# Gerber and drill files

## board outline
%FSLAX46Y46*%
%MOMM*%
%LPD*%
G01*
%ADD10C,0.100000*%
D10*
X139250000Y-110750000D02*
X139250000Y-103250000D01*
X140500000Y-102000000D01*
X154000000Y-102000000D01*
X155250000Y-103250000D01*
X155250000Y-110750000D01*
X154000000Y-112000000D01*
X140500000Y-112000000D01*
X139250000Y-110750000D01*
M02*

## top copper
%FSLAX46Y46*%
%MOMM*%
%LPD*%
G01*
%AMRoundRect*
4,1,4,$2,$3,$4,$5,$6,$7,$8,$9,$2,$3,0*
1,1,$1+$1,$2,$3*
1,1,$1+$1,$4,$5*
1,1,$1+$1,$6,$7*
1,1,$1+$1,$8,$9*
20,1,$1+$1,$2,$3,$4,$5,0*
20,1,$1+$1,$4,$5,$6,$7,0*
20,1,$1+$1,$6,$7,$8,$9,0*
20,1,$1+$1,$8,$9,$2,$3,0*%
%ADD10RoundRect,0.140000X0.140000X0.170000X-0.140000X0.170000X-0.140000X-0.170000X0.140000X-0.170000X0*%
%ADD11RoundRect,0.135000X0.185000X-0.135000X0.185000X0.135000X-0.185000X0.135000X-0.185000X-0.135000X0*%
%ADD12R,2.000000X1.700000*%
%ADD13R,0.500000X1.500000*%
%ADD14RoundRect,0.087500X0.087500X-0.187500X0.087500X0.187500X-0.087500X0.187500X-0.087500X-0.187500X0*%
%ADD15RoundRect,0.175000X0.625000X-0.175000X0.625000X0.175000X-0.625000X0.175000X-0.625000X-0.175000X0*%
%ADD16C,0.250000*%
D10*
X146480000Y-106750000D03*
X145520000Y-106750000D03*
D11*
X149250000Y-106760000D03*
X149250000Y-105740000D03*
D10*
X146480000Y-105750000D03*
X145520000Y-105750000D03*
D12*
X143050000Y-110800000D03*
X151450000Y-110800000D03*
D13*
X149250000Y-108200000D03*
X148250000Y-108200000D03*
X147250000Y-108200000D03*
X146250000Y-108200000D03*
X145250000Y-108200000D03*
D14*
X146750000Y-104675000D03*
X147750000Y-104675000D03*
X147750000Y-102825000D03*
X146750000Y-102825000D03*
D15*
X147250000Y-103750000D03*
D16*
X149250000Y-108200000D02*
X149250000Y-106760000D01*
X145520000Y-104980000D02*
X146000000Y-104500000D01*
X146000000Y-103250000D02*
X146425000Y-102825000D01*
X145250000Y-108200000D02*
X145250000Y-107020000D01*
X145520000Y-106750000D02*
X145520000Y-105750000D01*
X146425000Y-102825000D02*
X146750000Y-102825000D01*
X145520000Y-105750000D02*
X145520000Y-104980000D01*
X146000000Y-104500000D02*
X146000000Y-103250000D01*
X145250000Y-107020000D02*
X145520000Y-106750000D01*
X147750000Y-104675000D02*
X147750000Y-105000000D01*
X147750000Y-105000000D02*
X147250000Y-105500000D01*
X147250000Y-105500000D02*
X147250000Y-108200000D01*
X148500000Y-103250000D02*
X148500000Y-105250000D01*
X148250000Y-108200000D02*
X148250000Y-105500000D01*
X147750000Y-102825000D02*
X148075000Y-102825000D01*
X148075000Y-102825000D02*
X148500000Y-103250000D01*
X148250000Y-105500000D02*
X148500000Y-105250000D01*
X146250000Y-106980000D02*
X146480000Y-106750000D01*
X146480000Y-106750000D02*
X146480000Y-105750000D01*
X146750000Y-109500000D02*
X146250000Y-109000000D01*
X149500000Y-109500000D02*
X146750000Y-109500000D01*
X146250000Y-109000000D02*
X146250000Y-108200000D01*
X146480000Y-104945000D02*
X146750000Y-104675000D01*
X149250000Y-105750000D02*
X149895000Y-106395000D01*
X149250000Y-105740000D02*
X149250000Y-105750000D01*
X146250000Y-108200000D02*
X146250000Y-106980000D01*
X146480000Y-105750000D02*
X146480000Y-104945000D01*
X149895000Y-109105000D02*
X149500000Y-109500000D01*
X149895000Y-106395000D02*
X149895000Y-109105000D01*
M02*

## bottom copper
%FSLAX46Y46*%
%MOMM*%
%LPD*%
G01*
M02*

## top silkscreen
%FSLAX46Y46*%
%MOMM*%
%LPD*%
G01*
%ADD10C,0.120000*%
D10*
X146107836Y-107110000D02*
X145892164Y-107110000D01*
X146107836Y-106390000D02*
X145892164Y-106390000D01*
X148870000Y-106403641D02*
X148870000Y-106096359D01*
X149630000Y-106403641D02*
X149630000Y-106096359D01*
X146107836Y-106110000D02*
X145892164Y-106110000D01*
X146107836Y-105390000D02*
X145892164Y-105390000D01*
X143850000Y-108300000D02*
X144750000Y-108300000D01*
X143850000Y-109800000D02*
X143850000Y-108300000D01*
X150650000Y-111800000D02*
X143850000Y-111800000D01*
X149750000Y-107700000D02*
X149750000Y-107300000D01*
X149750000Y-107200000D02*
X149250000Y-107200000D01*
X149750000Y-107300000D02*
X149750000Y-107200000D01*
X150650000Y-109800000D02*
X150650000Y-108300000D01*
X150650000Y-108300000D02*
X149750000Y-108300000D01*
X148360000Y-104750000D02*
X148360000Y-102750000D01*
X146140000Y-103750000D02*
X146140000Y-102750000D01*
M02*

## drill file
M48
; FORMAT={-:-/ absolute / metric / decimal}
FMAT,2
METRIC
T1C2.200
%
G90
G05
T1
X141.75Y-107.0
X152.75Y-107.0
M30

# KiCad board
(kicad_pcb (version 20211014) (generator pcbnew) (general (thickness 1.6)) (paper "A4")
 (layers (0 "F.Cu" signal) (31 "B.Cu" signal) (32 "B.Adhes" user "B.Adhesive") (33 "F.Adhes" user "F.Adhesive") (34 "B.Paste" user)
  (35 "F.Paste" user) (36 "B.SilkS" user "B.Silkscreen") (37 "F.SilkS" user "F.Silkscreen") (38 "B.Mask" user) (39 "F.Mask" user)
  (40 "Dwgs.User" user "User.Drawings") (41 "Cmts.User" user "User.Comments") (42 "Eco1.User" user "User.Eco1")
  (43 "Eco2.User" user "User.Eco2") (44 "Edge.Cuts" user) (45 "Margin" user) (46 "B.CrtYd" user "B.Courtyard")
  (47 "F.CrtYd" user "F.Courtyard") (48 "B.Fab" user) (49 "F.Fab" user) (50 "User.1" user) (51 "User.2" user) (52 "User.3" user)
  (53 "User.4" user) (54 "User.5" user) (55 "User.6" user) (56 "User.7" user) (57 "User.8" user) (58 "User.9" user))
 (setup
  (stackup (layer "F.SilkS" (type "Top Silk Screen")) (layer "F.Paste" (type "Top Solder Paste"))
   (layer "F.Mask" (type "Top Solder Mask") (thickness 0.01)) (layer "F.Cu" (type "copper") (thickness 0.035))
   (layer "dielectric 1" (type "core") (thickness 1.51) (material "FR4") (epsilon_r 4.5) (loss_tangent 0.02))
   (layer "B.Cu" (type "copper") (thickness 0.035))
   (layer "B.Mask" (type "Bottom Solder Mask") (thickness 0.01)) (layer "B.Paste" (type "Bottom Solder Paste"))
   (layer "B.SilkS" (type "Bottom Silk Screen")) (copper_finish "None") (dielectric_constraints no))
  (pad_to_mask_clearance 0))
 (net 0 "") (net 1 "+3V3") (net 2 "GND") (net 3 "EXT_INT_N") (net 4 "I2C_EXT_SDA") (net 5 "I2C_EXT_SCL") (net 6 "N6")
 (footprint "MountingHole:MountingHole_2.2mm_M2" (layer "F.Cu") (at 152.75 107)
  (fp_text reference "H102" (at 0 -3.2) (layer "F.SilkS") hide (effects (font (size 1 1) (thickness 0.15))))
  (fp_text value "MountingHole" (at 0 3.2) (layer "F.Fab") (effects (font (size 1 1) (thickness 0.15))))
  (pad "" np_thru_hole circle (at 0 0) (size 2.2 2.2) (drill 2.2) (layers *.Cu *.Mask)))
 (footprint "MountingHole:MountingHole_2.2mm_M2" (layer "F.Cu") (at 141.75 107)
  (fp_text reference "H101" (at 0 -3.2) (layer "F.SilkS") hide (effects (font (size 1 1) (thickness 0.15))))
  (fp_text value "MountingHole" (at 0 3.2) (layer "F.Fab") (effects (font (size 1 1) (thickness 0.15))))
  (pad "" np_thru_hole circle (at 0 0) (size 2.2 2.2) (drill 2.2) (layers *.Cu *.Mask)))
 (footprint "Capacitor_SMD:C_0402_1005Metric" (layer "F.Cu") (at 146 106.75 180)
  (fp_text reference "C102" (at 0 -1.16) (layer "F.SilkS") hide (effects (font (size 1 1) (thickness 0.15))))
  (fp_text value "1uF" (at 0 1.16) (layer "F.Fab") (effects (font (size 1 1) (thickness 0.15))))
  (fp_line (start -0.107836 -0.36) (end 0.107836 -0.36) (layer "F.SilkS") (width 0.12))
  (fp_line (start -0.107836 0.36) (end 0.107836 0.36) (layer "F.SilkS") (width 0.12))
  (pad "1" smd roundrect (at -0.48 0 180) (size 0.56 0.62) (layers "F.Cu" "F.Paste" "F.Mask") (roundrect_rratio 0.25) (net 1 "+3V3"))
  (pad "2" smd roundrect (at 0.48 0 180) (size 0.56 0.62) (layers "F.Cu" "F.Paste" "F.Mask") (roundrect_rratio 0.25) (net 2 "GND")))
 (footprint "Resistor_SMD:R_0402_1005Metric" (layer "F.Cu") (at 149.25 106.25 90)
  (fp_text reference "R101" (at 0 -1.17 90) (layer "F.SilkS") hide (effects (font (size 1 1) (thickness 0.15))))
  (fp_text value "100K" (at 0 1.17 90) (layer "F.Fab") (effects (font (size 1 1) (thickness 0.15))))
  (fp_line (start -0.153641 -0.38) (end 0.153641 -0.38) (layer "F.SilkS") (width 0.12))
  (fp_line (start -0.153641 0.38) (end 0.153641 0.38) (layer "F.SilkS") (width 0.12))
  (pad "1" smd roundrect (at -0.51 0 90) (size 0.54 0.64) (layers "F.Cu" "F.Paste" "F.Mask") (roundrect_rratio 0.25) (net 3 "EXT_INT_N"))
  (pad "2" smd roundrect (at 0.51 0 90) (size 0.54 0.64) (layers "F.Cu" "F.Paste" "F.Mask") (roundrect_rratio 0.25) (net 1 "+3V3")))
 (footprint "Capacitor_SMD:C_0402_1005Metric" (layer "F.Cu") (at 146 105.75 180)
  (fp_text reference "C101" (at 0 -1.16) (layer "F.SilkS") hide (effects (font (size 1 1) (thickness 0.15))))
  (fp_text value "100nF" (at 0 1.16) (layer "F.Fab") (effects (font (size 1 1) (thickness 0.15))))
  (fp_line (start -0.107836 -0.36) (end 0.107836 -0.36) (layer "F.SilkS") (width 0.12))
  (fp_line (start -0.107836 0.36) (end 0.107836 0.36) (layer "F.SilkS") (width 0.12))
  (pad "1" smd roundrect (at -0.48 0 180) (size 0.56 0.62) (layers "F.Cu" "F.Paste" "F.Mask") (roundrect_rratio 0.25) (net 1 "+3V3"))
  (pad "2" smd roundrect (at 0.48 0 180) (size 0.56 0.62) (layers "F.Cu" "F.Paste" "F.Mask") (roundrect_rratio 0.25) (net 2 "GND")))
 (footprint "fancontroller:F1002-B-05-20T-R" (layer "F.Cu") (at 147.25 109.5 180)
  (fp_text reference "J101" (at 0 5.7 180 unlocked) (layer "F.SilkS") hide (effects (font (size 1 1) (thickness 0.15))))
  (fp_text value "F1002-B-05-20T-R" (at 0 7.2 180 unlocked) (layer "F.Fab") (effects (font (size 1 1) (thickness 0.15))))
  (fp_line (start 3.4 1.2) (end 2.5 1.2) (layer "F.SilkS") (width 0.12))
  (fp_line (start 3.4 -0.3) (end 3.4 1.2) (layer "F.SilkS") (width 0.12))
  (fp_line (start -3.4 -2.3) (end 3.4 -2.3) (layer "F.SilkS") (width 0.12))
  (fp_line (start -2.5 1.8) (end -2.5 2.2) (layer "F.SilkS") (width 0.12))
  (fp_line (start -2.5 2.3) (end -2 2.3) (layer "F.SilkS") (width 0.12))
  (fp_line (start -2.5 2.2) (end -2.5 2.3) (layer "F.SilkS") (width 0.12))
  (fp_line (start -3.4 -0.3) (end -3.4 1.2) (layer "F.SilkS") (width 0.12))
  (fp_line (start -3.4 1.2) (end -2.5 1.2) (layer "F.SilkS") (width 0.12))
  (pad "" smd rect (at 4.2 -1.3 270) (size 1.7 2) (layers "F.Cu" "F.Paste" "F.Mask"))
  (pad "" smd rect (at -4.2 -1.3 270) (size 1.7 2) (layers "F.Cu" "F.Paste" "F.Mask"))
  (pad "1" smd rect (at -2 1.3 270) (size 1.5 0.5) (layers "F.Cu" "F.Paste" "F.Mask") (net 3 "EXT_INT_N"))
  (pad "2" smd rect (at -1 1.3 270) (size 1.5 0.5) (layers "F.Cu" "F.Paste" "F.Mask") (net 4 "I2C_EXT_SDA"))
  (pad "3" smd rect (at 0 1.3 270) (size 1.5 0.5) (layers "F.Cu" "F.Paste" "F.Mask") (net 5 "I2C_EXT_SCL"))
  (pad "4" smd rect (at 1 1.3 270) (size 1.5 0.5) (layers "F.Cu" "F.Paste" "F.Mask") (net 1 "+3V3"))
  (pad "5" smd rect (at 2 1.3 270) (size 1.5 0.5) (layers "F.Cu" "F.Paste" "F.Mask") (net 2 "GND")))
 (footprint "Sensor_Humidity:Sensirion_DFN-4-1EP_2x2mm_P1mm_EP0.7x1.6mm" (layer "F.Cu") (at 147.25 103.75 90)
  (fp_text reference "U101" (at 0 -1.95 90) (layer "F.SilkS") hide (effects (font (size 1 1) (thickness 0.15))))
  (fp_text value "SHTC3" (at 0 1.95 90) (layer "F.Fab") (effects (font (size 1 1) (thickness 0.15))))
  (fp_line (start -1 1.11) (end 1 1.11) (layer "F.SilkS") (width 0.12))
  (fp_line (start 0 -1.11) (end 1 -1.11) (layer "F.SilkS") (width 0.12))
  (pad "" smd roundrect (at 1.025 -0.5 270) (size 0.55 0.35) (layers "F.Paste") (roundrect_rratio 0.25))
  (pad "" smd roundrect (at -1.025 0.5 90) (size 0.55 0.35) (layers "F.Paste") (roundrect_rratio 0.25))
  (pad "" smd roundrect (at 0 0 90) (size 0.5 1.4) (layers "F.Paste") (roundrect_rratio 0.25))
  (pad "" smd roundrect (at 1.025 0.5 270) (size 0.55 0.35) (layers "F.Paste") (roundrect_rratio 0.25))
  (pad "" smd roundrect (at -1.025 -0.5 90) (size 0.55 0.35) (layers "F.Paste") (roundrect_rratio 0.25))
  (pad "1" smd roundrect (at -0.925 -0.5 90) (size 0.55 0.35) (layers "F.Cu" "F.Mask") (roundrect_rratio 0.25) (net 1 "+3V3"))
  (pad "2" smd roundrect (at -0.925 0.5 90) (size 0.55 0.35) (layers "F.Cu" "F.Mask") (roundrect_rratio 0.25) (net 5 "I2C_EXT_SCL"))
  (pad "3" smd roundrect (at 0.925 0.5 90) (size 0.55 0.35) (layers "F.Cu" "F.Mask") (roundrect_rratio 0.25) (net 4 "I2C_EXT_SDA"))
  (pad "4" smd roundrect (at 0.925 -0.5 90) (size 0.55 0.35) (layers "F.Cu" "F.Mask") (roundrect_rratio 0.25) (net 2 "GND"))
  (pad "5" smd roundrect (at 0 0 90) (size 0.7 1.6) (layers "F.Cu" "F.Mask") (roundrect_rratio 0.25) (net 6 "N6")))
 (gr_poly
  (pts (xy 139.25 110.75) (xy 139.25 103.25) (xy 140.5 102) (xy 154 102) (xy 155.25 103.25) (xy 155.25 110.75) (xy 154 112) (xy 140.5 112))
  (layer "Edge.Cuts") (width 0.1) (fill none))
 (segment (start 149.25 108.2) (end 149.25 106.76) (width 0.25) (layer "F.Cu") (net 3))
 (segment (start 145.52 104.98) (end 146 104.5) (width 0.25) (layer "F.Cu") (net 2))
 (segment (start 146 103.25) (end 146.425 102.825) (width 0.25) (layer "F.Cu") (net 2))
 (segment (start 145.25 108.2) (end 145.25 107.02) (width 0.25) (layer "F.Cu") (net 2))
 (segment (start 145.52 106.75) (end 145.52 105.75) (width 0.25) (layer "F.Cu") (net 2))
 (segment (start 146.425 102.825) (end 146.75 102.825) (width 0.25) (layer "F.Cu") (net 2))
 (segment (start 145.52 105.75) (end 145.52 104.98) (width 0.25) (layer "F.Cu") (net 2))
 (segment (start 146 104.5) (end 146 103.25) (width 0.25) (layer "F.Cu") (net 2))
 (segment (start 145.25 107.02) (end 145.52 106.75) (width 0.25) (layer "F.Cu") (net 2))
 (segment (start 147.75 104.675) (end 147.75 105) (width 0.25) (layer "F.Cu") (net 5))
 (segment (start 147.75 105) (end 147.25 105.5) (width 0.25) (layer "F.Cu") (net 5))
 (segment (start 147.25 105.5) (end 147.25 108.2) (width 0.25) (layer "F.Cu") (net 5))
 (segment (start 148.5 103.25) (end 148.5 105.25) (width 0.25) (layer "F.Cu") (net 4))
 (segment (start 148.25 108.2) (end 148.25 105.5) (width 0.25) (layer "F.Cu") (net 4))
 (segment (start 147.75 102.825) (end 148.075 102.825) (width 0.25) (layer "F.Cu") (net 4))
 (segment (start 148.075 102.825) (end 148.5 103.25) (width 0.25) (layer "F.Cu") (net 4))
 (segment (start 148.25 105.5) (end 148.5 105.25) (width 0.25) (layer "F.Cu") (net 4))
 (segment (start 146.25 106.98) (end 146.48 106.75) (width 0.25) (layer "F.Cu") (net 1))
 (segment (start 146.48 106.75) (end 146.48 105.75) (width 0.25) (layer "F.Cu") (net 1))
 (segment (start 146.75 109.5) (end 146.25 109) (width 0.25) (layer "F.Cu") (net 1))
 (segment (start 149.5 109.5) (end 146.75 109.5) (width 0.25) (layer "F.Cu") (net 1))
 (segment (start 146.25 109) (end 146.25 108.2) (width 0.25) (layer "F.Cu") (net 1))
 (segment (start 146.48 104.945) (end 146.75 104.675) (width 0.25) (layer "F.Cu") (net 1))
 (segment (start 149.25 105.75) (end 149.895 106.395) (width 0.25) (layer "F.Cu") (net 1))
 (segment (start 149.25 105.74) (end 149.25 105.75) (width 0.25) (layer "F.Cu") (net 1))
 (segment (start 146.25 108.2) (end 146.25 106.98) (width 0.25) (layer "F.Cu") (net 1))
 (segment (start 146.48 105.75) (end 146.48 104.945) (width 0.25) (layer "F.Cu") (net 1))
 (segment (start 149.895 109.105) (end 149.5 109.5) (width 0.25) (layer "F.Cu") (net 1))
 (segment (start 149.895 106.395) (end 149.895 109.105) (width 0.25) (layer "F.Cu") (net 1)))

